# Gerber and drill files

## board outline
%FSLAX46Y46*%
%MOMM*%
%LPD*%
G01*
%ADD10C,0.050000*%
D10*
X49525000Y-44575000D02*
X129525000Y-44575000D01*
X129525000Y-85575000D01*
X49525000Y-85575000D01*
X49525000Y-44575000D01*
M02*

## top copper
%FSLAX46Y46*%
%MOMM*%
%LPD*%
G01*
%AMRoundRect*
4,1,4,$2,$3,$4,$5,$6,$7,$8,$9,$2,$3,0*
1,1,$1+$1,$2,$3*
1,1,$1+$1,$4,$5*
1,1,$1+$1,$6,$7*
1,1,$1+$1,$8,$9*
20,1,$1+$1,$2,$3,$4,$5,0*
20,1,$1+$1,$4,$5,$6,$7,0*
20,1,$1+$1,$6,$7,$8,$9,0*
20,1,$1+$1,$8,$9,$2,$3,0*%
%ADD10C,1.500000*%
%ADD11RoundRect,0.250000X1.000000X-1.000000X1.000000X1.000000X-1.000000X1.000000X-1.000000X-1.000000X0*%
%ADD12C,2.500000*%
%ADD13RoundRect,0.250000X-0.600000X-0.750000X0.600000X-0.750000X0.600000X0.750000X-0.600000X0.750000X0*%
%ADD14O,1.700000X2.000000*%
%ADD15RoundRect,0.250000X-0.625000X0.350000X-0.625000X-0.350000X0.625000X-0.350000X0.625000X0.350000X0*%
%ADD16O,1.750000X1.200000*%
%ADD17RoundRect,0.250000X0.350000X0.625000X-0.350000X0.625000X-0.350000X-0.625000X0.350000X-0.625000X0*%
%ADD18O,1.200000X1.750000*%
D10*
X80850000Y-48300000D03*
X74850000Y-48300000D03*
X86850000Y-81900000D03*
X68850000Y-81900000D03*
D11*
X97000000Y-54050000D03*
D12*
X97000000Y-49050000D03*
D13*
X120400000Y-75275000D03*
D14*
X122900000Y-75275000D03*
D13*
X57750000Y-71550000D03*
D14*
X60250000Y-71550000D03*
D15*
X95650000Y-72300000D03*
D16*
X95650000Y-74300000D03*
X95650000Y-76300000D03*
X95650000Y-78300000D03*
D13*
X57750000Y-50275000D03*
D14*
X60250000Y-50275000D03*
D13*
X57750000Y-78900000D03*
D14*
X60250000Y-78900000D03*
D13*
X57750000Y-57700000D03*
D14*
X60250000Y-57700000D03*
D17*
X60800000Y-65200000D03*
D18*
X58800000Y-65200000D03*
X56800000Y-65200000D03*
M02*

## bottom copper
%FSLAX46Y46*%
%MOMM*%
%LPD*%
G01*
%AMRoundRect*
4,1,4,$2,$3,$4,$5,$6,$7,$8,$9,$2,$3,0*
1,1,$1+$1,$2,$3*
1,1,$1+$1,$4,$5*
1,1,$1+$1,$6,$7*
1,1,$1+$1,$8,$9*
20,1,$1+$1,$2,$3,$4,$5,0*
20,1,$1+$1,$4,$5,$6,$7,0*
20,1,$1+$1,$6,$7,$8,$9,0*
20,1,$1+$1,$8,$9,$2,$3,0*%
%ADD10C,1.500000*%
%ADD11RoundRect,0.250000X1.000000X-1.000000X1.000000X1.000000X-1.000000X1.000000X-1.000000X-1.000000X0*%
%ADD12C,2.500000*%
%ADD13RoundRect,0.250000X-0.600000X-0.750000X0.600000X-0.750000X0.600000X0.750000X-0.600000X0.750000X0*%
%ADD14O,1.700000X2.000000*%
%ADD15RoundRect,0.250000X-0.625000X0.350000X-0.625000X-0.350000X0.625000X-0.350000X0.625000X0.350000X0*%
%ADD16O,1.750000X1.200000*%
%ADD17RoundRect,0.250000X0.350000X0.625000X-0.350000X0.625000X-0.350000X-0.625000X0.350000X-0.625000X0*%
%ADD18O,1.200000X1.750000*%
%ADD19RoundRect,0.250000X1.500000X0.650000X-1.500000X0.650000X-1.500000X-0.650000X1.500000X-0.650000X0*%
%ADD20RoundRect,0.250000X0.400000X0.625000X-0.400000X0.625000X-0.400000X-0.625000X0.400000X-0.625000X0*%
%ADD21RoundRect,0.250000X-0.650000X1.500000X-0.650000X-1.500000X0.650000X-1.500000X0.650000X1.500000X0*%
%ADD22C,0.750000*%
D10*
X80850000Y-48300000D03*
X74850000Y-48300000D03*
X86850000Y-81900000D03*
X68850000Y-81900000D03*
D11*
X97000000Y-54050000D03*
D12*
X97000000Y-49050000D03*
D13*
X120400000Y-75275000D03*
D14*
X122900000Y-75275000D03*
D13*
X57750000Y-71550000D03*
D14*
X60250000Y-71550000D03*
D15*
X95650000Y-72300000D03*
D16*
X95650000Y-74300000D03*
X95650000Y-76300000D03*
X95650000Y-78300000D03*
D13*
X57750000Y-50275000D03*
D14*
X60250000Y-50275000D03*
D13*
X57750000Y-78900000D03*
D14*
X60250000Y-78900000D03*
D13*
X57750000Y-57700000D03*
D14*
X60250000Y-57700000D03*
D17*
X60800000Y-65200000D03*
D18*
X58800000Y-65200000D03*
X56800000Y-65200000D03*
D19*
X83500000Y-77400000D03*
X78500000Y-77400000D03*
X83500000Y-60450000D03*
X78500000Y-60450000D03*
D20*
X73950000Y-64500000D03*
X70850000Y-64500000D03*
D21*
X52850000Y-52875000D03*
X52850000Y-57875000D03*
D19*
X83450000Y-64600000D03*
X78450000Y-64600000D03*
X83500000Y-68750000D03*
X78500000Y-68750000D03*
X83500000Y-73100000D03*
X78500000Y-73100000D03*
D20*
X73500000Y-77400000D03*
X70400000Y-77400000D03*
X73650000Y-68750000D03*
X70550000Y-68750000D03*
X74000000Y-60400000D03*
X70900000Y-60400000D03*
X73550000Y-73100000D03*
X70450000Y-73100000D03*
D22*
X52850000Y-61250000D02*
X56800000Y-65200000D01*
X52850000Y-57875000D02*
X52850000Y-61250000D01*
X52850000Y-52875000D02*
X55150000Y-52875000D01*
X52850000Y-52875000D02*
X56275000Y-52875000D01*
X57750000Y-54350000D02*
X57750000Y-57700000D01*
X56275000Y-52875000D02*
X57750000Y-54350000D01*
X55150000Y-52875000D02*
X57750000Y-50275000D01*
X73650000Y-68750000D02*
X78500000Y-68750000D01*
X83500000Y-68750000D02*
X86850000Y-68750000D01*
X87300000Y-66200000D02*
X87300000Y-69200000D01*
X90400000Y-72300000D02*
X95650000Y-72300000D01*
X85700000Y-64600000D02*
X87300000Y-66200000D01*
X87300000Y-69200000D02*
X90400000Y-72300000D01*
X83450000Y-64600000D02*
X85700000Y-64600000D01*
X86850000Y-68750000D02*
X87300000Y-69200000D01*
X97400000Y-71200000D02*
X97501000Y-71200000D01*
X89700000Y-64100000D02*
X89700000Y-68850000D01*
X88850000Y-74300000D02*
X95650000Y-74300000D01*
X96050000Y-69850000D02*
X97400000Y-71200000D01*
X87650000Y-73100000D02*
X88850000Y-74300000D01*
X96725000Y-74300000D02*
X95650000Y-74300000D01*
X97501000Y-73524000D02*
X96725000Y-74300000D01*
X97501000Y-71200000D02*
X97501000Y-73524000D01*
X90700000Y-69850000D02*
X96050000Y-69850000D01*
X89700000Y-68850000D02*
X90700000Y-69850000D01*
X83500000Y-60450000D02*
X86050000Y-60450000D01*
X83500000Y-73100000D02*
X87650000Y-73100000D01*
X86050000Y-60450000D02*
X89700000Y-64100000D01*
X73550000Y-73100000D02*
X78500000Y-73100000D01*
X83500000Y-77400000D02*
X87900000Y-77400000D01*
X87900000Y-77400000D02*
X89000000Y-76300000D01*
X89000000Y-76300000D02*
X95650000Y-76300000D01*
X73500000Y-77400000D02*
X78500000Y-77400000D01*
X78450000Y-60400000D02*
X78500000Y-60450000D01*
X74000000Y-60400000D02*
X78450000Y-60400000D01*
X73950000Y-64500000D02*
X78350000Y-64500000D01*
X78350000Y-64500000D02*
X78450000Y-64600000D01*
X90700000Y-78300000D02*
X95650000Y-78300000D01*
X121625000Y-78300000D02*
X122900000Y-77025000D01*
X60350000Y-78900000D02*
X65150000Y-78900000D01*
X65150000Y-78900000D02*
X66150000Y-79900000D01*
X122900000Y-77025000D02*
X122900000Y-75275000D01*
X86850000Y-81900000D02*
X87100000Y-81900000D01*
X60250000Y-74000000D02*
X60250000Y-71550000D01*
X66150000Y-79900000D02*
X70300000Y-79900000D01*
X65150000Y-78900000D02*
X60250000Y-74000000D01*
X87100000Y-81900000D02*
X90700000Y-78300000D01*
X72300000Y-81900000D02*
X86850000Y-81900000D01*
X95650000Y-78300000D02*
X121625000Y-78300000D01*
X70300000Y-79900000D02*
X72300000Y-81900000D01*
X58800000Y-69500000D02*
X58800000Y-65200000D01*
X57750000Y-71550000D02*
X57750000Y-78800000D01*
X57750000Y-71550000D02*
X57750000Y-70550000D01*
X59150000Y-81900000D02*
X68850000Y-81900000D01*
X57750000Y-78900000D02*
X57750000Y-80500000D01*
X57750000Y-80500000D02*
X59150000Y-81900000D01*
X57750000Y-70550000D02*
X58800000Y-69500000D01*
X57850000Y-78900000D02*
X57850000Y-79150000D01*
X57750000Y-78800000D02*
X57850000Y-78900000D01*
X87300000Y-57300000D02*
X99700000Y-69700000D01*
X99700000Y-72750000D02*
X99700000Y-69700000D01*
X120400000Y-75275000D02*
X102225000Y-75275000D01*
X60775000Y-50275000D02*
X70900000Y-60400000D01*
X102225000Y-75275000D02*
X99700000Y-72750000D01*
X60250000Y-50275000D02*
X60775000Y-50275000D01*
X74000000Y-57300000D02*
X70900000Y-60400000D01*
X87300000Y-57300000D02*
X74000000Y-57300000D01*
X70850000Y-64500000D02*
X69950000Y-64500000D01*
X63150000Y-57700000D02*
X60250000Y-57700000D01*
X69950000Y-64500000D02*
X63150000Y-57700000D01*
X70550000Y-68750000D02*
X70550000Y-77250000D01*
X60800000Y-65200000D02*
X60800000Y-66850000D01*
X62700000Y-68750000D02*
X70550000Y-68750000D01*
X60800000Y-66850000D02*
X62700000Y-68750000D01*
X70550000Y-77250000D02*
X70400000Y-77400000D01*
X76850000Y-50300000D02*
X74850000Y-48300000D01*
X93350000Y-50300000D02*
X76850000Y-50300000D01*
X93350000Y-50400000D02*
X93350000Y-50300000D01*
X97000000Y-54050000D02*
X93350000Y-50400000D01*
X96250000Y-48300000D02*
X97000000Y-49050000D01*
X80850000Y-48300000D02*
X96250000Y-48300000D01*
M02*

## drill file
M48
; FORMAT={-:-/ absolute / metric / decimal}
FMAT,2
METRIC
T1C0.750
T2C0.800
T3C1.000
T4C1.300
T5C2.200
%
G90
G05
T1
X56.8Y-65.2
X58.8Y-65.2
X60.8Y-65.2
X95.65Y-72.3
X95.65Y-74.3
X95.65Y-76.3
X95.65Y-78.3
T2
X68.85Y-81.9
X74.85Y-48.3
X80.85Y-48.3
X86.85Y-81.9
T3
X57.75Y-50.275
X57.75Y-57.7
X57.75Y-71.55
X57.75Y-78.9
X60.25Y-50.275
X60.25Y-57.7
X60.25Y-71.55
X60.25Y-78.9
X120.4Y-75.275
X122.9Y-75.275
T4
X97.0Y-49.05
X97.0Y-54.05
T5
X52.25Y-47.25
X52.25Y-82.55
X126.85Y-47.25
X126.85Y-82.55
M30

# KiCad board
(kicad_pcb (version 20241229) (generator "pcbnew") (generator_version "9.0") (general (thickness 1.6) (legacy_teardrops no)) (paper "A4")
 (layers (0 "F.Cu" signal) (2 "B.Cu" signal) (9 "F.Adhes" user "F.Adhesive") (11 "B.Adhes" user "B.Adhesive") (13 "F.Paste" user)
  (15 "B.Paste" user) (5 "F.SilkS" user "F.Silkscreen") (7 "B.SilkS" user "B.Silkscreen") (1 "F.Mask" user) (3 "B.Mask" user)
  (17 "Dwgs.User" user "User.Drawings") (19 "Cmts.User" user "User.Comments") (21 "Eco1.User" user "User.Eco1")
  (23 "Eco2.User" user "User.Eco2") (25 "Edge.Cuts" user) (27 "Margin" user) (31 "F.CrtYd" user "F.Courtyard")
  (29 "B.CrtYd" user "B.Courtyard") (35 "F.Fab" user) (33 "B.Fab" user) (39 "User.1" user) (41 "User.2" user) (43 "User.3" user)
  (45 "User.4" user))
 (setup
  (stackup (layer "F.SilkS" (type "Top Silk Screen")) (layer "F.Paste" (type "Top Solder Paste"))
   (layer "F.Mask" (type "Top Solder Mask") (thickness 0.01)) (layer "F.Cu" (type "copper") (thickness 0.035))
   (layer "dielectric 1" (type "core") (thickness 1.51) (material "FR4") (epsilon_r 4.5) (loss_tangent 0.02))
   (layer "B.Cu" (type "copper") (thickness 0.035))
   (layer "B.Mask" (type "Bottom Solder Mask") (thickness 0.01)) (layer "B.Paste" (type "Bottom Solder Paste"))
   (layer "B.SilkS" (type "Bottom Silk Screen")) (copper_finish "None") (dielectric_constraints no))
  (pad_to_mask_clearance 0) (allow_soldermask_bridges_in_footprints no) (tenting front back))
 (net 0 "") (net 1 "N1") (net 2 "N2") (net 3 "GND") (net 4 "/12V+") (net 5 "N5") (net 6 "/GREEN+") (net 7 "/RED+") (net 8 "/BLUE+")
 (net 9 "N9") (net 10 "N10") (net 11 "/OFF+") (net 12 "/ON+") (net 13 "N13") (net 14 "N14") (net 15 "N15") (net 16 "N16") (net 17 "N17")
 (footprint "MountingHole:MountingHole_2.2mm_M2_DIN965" (layer "F.Cu") (at 52.25 47.25)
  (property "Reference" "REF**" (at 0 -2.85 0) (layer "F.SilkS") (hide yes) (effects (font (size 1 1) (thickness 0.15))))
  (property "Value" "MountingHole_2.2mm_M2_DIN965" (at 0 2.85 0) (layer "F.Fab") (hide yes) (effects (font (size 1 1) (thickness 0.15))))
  (pad "" np_thru_hole circle (at 0 0) (size 2.2 2.2) (drill 2.2) (layers "*.Cu" "*.Mask")))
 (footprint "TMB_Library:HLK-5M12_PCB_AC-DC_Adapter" (layer "F.Cu") (at 77.85 65.1 -90)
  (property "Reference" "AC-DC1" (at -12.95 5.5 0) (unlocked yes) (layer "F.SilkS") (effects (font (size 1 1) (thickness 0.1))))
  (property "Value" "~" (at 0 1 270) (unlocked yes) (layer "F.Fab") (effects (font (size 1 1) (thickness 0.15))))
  (pad "1" thru_hole circle (at -16.8 -3 270) (size 1.5 1.5) (drill 0.8) (layers "*.Cu" "*.Mask") (remove_unused_layers yes)
   (keep_end_layers yes) (zone_layer_connections) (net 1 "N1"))
  (pad "2" thru_hole circle (at -16.8 3 270) (size 1.5 1.5) (drill 0.8) (layers "*.Cu" "*.Mask") (remove_unused_layers yes)
   (keep_end_layers yes) (zone_layer_connections) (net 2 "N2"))
  (pad "3" thru_hole circle (at 16.8 -9 270) (size 1.5 1.5) (drill 0.8) (layers "*.Cu" "*.Mask") (remove_unused_layers yes)
   (keep_end_layers yes) (zone_layer_connections) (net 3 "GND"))
  (pad "4" thru_hole circle (at 16.8 9 270) (size 1.5 1.5) (drill 0.8) (layers "*.Cu" "*.Mask") (remove_unused_layers yes)
   (keep_end_layers yes) (zone_layer_connections) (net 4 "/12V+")))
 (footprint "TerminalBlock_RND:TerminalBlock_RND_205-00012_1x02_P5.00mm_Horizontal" (layer "F.Cu") (at 97 54.05 90)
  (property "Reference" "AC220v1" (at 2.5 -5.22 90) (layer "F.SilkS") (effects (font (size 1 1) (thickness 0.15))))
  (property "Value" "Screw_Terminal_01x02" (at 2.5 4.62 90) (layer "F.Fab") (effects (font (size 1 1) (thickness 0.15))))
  (pad "1" thru_hole roundrect (at 0 0 90) (size 2.5 2.5) (drill 1.3) (layers "*.Cu" "*.Mask") (remove_unused_layers no)
   (roundrect_rratio 0.1) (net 2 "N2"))
  (pad "2" thru_hole circle (at 5 0 90) (size 2.5 2.5) (drill 1.3) (layers "*.Cu" "*.Mask") (remove_unused_layers no) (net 1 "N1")))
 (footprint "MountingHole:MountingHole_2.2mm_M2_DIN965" (layer "F.Cu") (at 52.25 82.55)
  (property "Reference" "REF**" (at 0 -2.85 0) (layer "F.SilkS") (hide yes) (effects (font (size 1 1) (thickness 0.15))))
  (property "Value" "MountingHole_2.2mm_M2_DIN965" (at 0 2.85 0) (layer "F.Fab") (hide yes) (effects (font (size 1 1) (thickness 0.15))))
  (pad "" np_thru_hole circle (at 0 0) (size 2.2 2.2) (drill 2.2) (layers "*.Cu" "*.Mask")))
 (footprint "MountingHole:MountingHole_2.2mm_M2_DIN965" (layer "F.Cu") (at 126.85 82.55)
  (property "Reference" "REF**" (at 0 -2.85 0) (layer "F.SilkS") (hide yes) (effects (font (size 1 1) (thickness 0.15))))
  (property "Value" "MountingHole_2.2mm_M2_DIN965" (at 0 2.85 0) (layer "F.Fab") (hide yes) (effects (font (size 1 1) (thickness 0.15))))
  (pad "" np_thru_hole circle (at 0 0) (size 2.2 2.2) (drill 2.2) (layers "*.Cu" "*.Mask")))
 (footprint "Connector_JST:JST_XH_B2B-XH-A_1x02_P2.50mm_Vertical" (layer "F.Cu") (at 120.4 75.275)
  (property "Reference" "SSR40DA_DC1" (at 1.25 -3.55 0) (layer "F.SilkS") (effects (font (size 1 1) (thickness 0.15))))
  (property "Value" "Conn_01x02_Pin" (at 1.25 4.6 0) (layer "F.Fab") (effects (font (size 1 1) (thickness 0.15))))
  (pad "1" thru_hole roundrect (at 0 0) (size 1.7 2) (drill 1) (layers "*.Cu" "*.Mask") (remove_unused_layers no)
   (roundrect_rratio 0.147059) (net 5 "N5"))
  (pad "2" thru_hole oval (at 2.5 0) (size 1.7 2) (drill 1) (layers "*.Cu" "*.Mask") (remove_unused_layers no) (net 3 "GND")))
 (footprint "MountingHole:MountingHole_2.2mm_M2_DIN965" (layer "F.Cu") (at 126.85 47.25)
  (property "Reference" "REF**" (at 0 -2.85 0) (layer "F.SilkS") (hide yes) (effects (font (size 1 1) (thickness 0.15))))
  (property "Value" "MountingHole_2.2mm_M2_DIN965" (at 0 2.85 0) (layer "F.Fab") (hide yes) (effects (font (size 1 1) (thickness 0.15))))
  (pad "" np_thru_hole circle (at 0 0) (size 2.2 2.2) (drill 2.2) (layers "*.Cu" "*.Mask")))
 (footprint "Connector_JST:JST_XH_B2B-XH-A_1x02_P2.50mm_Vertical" (layer "F.Cu") (at 57.75 71.55)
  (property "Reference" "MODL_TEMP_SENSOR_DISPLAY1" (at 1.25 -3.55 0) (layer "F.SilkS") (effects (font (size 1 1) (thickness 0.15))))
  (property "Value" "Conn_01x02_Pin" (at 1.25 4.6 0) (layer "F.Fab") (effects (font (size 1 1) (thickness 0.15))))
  (pad "1" thru_hole roundrect (at 0 0) (size 1.7 2) (drill 1) (layers "*.Cu" "*.Mask") (remove_unused_layers no)
   (roundrect_rratio 0.147059) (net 4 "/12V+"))
  (pad "2" thru_hole oval (at 2.5 0) (size 1.7 2) (drill 1) (layers "*.Cu" "*.Mask") (remove_unused_layers no) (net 3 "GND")))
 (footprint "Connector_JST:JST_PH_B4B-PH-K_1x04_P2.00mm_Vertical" (layer "F.Cu") (at 95.65 72.3 -90)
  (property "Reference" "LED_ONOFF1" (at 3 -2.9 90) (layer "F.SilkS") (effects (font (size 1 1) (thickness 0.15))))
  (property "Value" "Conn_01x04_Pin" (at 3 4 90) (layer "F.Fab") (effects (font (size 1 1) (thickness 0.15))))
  (pad "1" thru_hole roundrect (at 0 0 270) (size 1.2 1.75) (drill 0.75) (layers "*.Cu" "*.Mask") (remove_unused_layers no)
   (roundrect_rratio 0.208333) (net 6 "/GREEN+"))
  (pad "2" thru_hole oval (at 2 0 270) (size 1.2 1.75) (drill 0.75) (layers "*.Cu" "*.Mask") (remove_unused_layers no) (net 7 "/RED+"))
  (pad "3" thru_hole oval (at 4 0 270) (size 1.2 1.75) (drill 0.75) (layers "*.Cu" "*.Mask") (remove_unused_layers no) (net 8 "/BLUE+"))
  (pad "4" thru_hole oval (at 6 0 270) (size 1.2 1.75) (drill 0.75) (layers "*.Cu" "*.Mask") (remove_unused_layers no) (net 3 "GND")))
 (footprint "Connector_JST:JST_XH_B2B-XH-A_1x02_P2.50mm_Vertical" (layer "F.Cu") (at 57.75 50.275)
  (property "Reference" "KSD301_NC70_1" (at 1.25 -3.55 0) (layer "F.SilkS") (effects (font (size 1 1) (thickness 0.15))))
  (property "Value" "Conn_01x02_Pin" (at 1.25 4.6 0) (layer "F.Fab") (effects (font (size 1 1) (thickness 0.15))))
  (pad "1" thru_hole roundrect (at 0 0) (size 1.7 2) (drill 1) (layers "*.Cu" "*.Mask") (remove_unused_layers no)
   (roundrect_rratio 0.147059) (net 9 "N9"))
  (pad "2" thru_hole oval (at 2.5 0) (size 1.7 2) (drill 1) (layers "*.Cu" "*.Mask") (remove_unused_layers no) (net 5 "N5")))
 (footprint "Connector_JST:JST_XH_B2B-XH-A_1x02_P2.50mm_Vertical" (layer "F.Cu") (at 57.75 78.9)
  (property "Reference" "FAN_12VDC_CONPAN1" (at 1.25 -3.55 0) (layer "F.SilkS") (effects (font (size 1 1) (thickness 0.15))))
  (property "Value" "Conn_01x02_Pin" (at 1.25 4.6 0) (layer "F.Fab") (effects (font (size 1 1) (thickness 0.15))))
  (pad "1" thru_hole roundrect (at 0 0) (size 1.7 2) (drill 1) (layers "*.Cu" "*.Mask") (remove_unused_layers no)
   (roundrect_rratio 0.147059) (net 4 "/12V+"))
  (pad "2" thru_hole oval (at 2.5 0) (size 1.7 2) (drill 1) (layers "*.Cu" "*.Mask") (remove_unused_layers no) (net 3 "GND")))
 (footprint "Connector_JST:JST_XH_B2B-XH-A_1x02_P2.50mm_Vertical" (layer "F.Cu") (at 57.75 57.7)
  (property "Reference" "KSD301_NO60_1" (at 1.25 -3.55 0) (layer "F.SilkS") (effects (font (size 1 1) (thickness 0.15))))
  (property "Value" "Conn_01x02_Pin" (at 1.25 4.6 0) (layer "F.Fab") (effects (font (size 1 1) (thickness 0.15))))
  (pad "1" thru_hole roundrect (at 0 0) (size 1.7 2) (drill 1) (layers "*.Cu" "*.Mask") (remove_unused_layers no)
   (roundrect_rratio 0.147059) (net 9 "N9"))
  (pad "2" thru_hole oval (at 2.5 0) (size 1.7 2) (drill 1) (layers "*.Cu" "*.Mask") (remove_unused_layers no) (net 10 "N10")))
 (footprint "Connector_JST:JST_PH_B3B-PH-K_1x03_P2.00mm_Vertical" (layer "F.Cu") (at 60.8 65.2 180)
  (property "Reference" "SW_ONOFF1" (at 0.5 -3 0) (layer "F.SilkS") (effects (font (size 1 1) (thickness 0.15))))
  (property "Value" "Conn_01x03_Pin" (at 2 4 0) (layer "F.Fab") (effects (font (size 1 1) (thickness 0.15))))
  (pad "1" thru_hole roundrect (at 0 0 180) (size 1.2 1.75) (drill 0.75) (layers "*.Cu" "*.Mask") (remove_unused_layers no)
   (roundrect_rratio 0.208333) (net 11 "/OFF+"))
  (pad "2" thru_hole oval (at 2 0 180) (size 1.2 1.75) (drill 0.75) (layers "*.Cu" "*.Mask") (remove_unused_layers no) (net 4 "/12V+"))
  (pad "3" thru_hole oval (at 4 0 180) (size 1.2 1.75) (drill 0.75) (layers "*.Cu" "*.Mask") (remove_unused_layers no) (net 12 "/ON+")))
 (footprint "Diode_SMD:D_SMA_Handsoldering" (layer "B.Cu") (at 81 77.4 180)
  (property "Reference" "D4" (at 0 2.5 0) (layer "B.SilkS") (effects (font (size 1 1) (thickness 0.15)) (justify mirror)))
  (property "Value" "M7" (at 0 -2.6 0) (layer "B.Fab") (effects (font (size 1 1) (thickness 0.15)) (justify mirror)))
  (pad "1" smd roundrect (at -2.5 0 180) (size 3.5 1.8) (layers "B.Cu" "B.Mask" "B.Paste") (roundrect_rratio 0.1388888889) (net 8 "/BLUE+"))
  (pad "2" smd roundrect (at 2.5 0 180) (size 3.5 1.8) (layers "B.Cu" "B.Mask" "B.Paste") (roundrect_rratio 0.1388888889) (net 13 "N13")))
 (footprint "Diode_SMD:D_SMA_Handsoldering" (layer "B.Cu") (at 81 60.45 180)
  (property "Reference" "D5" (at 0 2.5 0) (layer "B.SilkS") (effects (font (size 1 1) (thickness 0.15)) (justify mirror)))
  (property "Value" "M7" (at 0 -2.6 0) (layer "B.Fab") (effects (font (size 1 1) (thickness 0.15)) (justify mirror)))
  (pad "1" smd roundrect (at -2.5 0 180) (size 3.5 1.8) (layers "B.Cu" "B.Mask" "B.Paste") (roundrect_rratio 0.1388888889) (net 7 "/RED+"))
  (pad "2" smd roundrect (at 2.5 0 180) (size 3.5 1.8) (layers "B.Cu" "B.Mask" "B.Paste") (roundrect_rratio 0.1388888889) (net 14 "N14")))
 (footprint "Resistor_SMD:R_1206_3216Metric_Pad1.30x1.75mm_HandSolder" (layer "B.Cu") (at 72.4 64.5 180)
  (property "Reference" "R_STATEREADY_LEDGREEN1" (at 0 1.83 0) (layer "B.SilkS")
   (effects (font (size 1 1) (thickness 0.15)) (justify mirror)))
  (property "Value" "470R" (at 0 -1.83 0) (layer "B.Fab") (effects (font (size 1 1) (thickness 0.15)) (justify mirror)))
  (pad "1" smd roundrect (at -1.55 0 180) (size 1.3 1.75) (layers "B.Cu" "B.Mask" "B.Paste") (roundrect_rratio 0.192308) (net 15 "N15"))
  (pad "2" smd roundrect (at 1.55 0 180) (size 1.3 1.75) (layers "B.Cu" "B.Mask" "B.Paste") (roundrect_rratio 0.192308) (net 10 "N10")))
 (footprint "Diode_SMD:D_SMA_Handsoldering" (layer "B.Cu") (at 52.85 55.375 -90)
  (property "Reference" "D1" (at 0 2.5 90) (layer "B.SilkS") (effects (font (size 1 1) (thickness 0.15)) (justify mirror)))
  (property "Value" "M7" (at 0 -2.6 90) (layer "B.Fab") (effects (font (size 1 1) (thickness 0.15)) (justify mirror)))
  (pad "1" smd roundrect (at -2.5 0 270) (size 3.5 1.8) (layers "B.Cu" "B.Mask" "B.Paste") (roundrect_rratio 0.1388888889) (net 9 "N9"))
  (pad "2" smd roundrect (at 2.5 0 270) (size 3.5 1.8) (layers "B.Cu" "B.Mask" "B.Paste") (roundrect_rratio 0.1388888889) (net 12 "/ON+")))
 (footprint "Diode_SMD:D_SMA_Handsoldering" (layer "B.Cu") (at 80.95 64.6 180)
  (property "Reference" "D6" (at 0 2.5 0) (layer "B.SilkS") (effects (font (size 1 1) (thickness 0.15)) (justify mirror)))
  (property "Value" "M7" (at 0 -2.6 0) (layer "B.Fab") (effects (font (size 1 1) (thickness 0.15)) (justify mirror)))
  (pad "1" smd roundrect (at -2.5 0 180) (size 3.5 1.8) (layers "B.Cu" "B.Mask" "B.Paste") (roundrect_rratio 0.1388888889) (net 6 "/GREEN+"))
  (pad "2" smd roundrect (at 2.5 0 180) (size 3.5 1.8) (layers "B.Cu" "B.Mask" "B.Paste") (roundrect_rratio 0.1388888889) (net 15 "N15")))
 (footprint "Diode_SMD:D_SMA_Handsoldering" (layer "B.Cu") (at 81 68.75 180)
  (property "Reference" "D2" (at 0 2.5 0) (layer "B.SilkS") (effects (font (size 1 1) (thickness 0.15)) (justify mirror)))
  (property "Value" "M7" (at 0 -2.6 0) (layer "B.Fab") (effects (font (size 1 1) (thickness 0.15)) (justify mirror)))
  (pad "1" smd roundrect (at -2.5 0 180) (size 3.5 1.8) (layers "B.Cu" "B.Mask" "B.Paste") (roundrect_rratio 0.1388888889) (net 6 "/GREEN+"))
  (pad "2" smd roundrect (at 2.5 0 180) (size 3.5 1.8) (layers "B.Cu" "B.Mask" "B.Paste") (roundrect_rratio 0.1388888889) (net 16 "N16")))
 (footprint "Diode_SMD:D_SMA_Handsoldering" (layer "B.Cu") (at 81 73.1 180)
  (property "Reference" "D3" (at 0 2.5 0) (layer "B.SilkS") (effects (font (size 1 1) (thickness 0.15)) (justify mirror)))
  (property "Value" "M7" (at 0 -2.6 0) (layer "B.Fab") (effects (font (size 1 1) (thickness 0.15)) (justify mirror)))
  (pad "1" smd roundrect (at -2.5 0 180) (size 3.5 1.8) (layers "B.Cu" "B.Mask" "B.Paste") (roundrect_rratio 0.1388888889) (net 7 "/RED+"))
  (pad "2" smd roundrect (at 2.5 0 180) (size 3.5 1.8) (layers "B.Cu" "B.Mask" "B.Paste") (roundrect_rratio 0.1388888889) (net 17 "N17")))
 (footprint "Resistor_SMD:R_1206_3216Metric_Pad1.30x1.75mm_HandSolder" (layer "B.Cu") (at 71.95 77.4 180)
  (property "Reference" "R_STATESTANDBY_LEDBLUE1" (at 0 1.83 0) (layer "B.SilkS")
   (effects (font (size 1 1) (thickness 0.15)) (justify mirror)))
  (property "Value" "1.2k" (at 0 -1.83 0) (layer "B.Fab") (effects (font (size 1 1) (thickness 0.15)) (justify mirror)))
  (pad "1" smd roundrect (at -1.55 0 180) (size 1.3 1.75) (layers "B.Cu" "B.Mask" "B.Paste") (roundrect_rratio 0.192308) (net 13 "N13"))
  (pad "2" smd roundrect (at 1.55 0 180) (size 1.3 1.75) (layers "B.Cu" "B.Mask" "B.Paste") (roundrect_rratio 0.192308) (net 11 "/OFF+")))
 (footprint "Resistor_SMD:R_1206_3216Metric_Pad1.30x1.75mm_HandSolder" (layer "B.Cu") (at 72.1 68.75 180)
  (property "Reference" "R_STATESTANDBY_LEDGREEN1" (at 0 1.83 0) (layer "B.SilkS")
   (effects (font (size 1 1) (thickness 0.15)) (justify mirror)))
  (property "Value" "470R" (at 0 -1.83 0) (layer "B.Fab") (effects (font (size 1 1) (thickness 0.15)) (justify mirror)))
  (pad "1" smd roundrect (at -1.55 0 180) (size 1.3 1.75) (layers "B.Cu" "B.Mask" "B.Paste") (roundrect_rratio 0.192308) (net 16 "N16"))
  (pad "2" smd roundrect (at 1.55 0 180) (size 1.3 1.75) (layers "B.Cu" "B.Mask" "B.Paste") (roundrect_rratio 0.192308) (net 11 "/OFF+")))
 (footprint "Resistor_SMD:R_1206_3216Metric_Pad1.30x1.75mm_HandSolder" (layer "B.Cu") (at 72.45 60.4 180)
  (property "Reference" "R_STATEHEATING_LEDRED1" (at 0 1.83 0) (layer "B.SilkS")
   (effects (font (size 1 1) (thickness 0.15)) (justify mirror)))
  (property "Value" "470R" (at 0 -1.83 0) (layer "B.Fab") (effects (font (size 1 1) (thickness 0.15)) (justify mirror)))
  (pad "1" smd roundrect (at -1.55 0 180) (size 1.3 1.75) (layers "B.Cu" "B.Mask" "B.Paste") (roundrect_rratio 0.192308) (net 14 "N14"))
  (pad "2" smd roundrect (at 1.55 0 180) (size 1.3 1.75) (layers "B.Cu" "B.Mask" "B.Paste") (roundrect_rratio 0.192308) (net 5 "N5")))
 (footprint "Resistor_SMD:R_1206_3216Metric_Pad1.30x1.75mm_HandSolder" (layer "B.Cu") (at 72 73.1 180)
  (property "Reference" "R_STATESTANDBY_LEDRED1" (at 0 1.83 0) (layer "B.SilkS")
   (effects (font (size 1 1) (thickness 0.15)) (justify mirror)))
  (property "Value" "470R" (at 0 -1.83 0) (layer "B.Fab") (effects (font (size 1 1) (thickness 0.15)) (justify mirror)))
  (pad "1" smd roundrect (at -1.55 0 180) (size 1.3 1.75) (layers "B.Cu" "B.Mask" "B.Paste") (roundrect_rratio 0.192308) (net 17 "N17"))
  (pad "2" smd roundrect (at 1.55 0 180) (size 1.3 1.75) (layers "B.Cu" "B.Mask" "B.Paste") (roundrect_rratio 0.192308) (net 11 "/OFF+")))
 (gr_rect (start 49.525 44.575) (end 129.525 85.575) (stroke (width 0.05) (type solid)) (fill no) (layer "Edge.Cuts"))
 (segment (start 52.85 61.25) (end 56.8 65.2) (width 0.75) (layer "B.Cu") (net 12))
 (segment (start 52.85 57.875) (end 52.85 61.25) (width 0.75) (layer "B.Cu") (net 12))
 (segment (start 52.85 52.875) (end 55.15 52.875) (width 0.75) (layer "B.Cu") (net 9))
 (segment (start 52.85 52.875) (end 56.275 52.875) (width 0.75) (layer "B.Cu") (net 9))
 (segment (start 57.75 54.35) (end 57.75 57.7) (width 0.75) (layer "B.Cu") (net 9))
 (segment (start 56.275 52.875) (end 57.75 54.35) (width 0.75) (layer "B.Cu") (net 9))
 (segment (start 55.15 52.875) (end 57.75 50.275) (width 0.75) (layer "B.Cu") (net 9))
 (segment (start 73.65 68.75) (end 78.5 68.75) (width 0.75) (layer "B.Cu") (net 16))
 (segment (start 83.5 68.75) (end 86.85 68.75) (width 0.75) (layer "B.Cu") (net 6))
 (segment (start 87.3 66.2) (end 87.3 69.2) (width 0.75) (layer "B.Cu") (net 6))
 (segment (start 90.4 72.3) (end 95.65 72.3) (width 0.75) (layer "B.Cu") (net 6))
 (segment (start 85.7 64.6) (end 87.3 66.2) (width 0.75) (layer "B.Cu") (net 6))
 (segment (start 87.3 69.2) (end 90.4 72.3) (width 0.75) (layer "B.Cu") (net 6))
 (segment (start 83.45 64.6) (end 85.7 64.6) (width 0.75) (layer "B.Cu") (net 6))
 (segment (start 86.85 68.75) (end 87.3 69.2) (width 0.75) (layer "B.Cu") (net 6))
 (segment (start 97.4 71.2) (end 97.501 71.2) (width 0.75) (layer "B.Cu") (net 7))
 (segment (start 89.7 64.1) (end 89.7 68.85) (width 0.75) (layer "B.Cu") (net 7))
 (segment (start 88.85 74.3) (end 95.65 74.3) (width 0.75) (layer "B.Cu") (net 7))
 (segment (start 96.05 69.85) (end 97.4 71.2) (width 0.75) (layer "B.Cu") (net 7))
 (segment (start 87.65 73.1) (end 88.85 74.3) (width 0.75) (layer "B.Cu") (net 7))
 (segment (start 96.725 74.3) (end 95.65 74.3) (width 0.75) (layer "B.Cu") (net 7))
 (segment (start 97.501 73.524) (end 96.725 74.3) (width 0.75) (layer "B.Cu") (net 7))
 (segment (start 97.501 71.2) (end 97.501 73.524) (width 0.75) (layer "B.Cu") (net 7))
 (segment (start 90.7 69.85) (end 96.05 69.85) (width 0.75) (layer "B.Cu") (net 7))
 (segment (start 89.7 68.85) (end 90.7 69.85) (width 0.75) (layer "B.Cu") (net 7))
 (segment (start 83.5 60.45) (end 86.05 60.45) (width 0.75) (layer "B.Cu") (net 7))
 (segment (start 83.5 73.1) (end 87.65 73.1) (width 0.75) (layer "B.Cu") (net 7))
 (segment (start 86.05 60.45) (end 89.7 64.1) (width 0.75) (layer "B.Cu") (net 7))
 (segment (start 73.55 73.1) (end 78.5 73.1) (width 0.75) (layer "B.Cu") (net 17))
 (segment (start 83.5 77.4) (end 87.9 77.4) (width 0.75) (layer "B.Cu") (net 8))
 (segment (start 87.9 77.4) (end 89 76.3) (width 0.75) (layer "B.Cu") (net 8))
 (segment (start 89 76.3) (end 95.65 76.3) (width 0.75) (layer "B.Cu") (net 8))
 (segment (start 73.5 77.4) (end 78.5 77.4) (width 0.75) (layer "B.Cu") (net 13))
 (segment (start 78.45 60.4) (end 78.5 60.45) (width 0.75) (layer "B.Cu") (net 14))
 (segment (start 74 60.4) (end 78.45 60.4) (width 0.75) (layer "B.Cu") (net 14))
 (segment (start 73.95 64.5) (end 78.35 64.5) (width 0.75) (layer "B.Cu") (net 15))
 (segment (start 78.35 64.5) (end 78.45 64.6) (width 0.75) (layer "B.Cu") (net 15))
 (segment (start 90.7 78.3) (end 95.65 78.3) (width 0.75) (layer "B.Cu") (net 3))
 (segment (start 121.625 78.3) (end 122.9 77.025) (width 0.75) (layer "B.Cu") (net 3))
 (segment (start 60.35 78.9) (end 65.15 78.9) (width 0.75) (layer "B.Cu") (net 3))
 (segment (start 65.15 78.9) (end 66.15 79.9) (width 0.75) (layer "B.Cu") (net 3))
 (segment (start 122.9 77.025) (end 122.9 75.275) (width 0.75) (layer "B.Cu") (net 3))
 (segment (start 86.85 81.9) (end 87.1 81.9) (width 0.75) (layer "B.Cu") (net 3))
 (segment (start 60.25 74) (end 60.25 71.55) (width 0.75) (layer "B.Cu") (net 3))
 (segment (start 66.15 79.9) (end 70.3 79.9) (width 0.75) (layer "B.Cu") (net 3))
 (segment (start 65.15 78.9) (end 60.25 74) (width 0.75) (layer "B.Cu") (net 3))
 (segment (start 87.1 81.9) (end 90.7 78.3) (width 0.75) (layer "B.Cu") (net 3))
 (segment (start 72.3 81.9) (end 86.85 81.9) (width 0.75) (layer "B.Cu") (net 3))
 (segment (start 95.65 78.3) (end 121.625 78.3) (width 0.75) (layer "B.Cu") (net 3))
 (segment (start 70.3 79.9) (end 72.3 81.9) (width 0.75) (layer "B.Cu") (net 3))
 (segment (start 58.8 69.5) (end 58.8 65.2) (width 0.75) (layer "B.Cu") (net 4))
 (segment (start 57.75 71.55) (end 57.75 78.8) (width 0.75) (layer "B.Cu") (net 4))
 (segment (start 57.75 71.55) (end 57.75 70.55) (width 0.75) (layer "B.Cu") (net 4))
 (segment (start 59.15 81.9) (end 68.85 81.9) (width 0.75) (layer "B.Cu") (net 4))
 (segment (start 57.75 78.9) (end 57.75 80.5) (width 0.75) (layer "B.Cu") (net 4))
 (segment (start 57.75 80.5) (end 59.15 81.9) (width 0.75) (layer "B.Cu") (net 4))
 (segment (start 57.75 70.55) (end 58.8 69.5) (width 0.75) (layer "B.Cu") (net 4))
 (segment (start 57.85 78.9) (end 57.85 79.15) (width 0.75) (layer "B.Cu") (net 4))
 (segment (start 57.75 78.8) (end 57.85 78.9) (width 0.75) (layer "B.Cu") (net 4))
 (segment (start 87.3 57.3) (end 99.7 69.7) (width 0.75) (layer "B.Cu") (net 5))
 (segment (start 99.7 72.75) (end 99.7 69.7) (width 0.75) (layer "B.Cu") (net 5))
 (segment (start 120.4 75.275) (end 102.225 75.275) (width 0.75) (layer "B.Cu") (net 5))
 (segment (start 60.775 50.275) (end 70.9 60.4) (width 0.75) (layer "B.Cu") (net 5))
 (segment (start 102.225 75.275) (end 99.7 72.75) (width 0.75) (layer "B.Cu") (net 5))
 (segment (start 60.25 50.275) (end 60.775 50.275) (width 0.75) (layer "B.Cu") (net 5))
 (segment (start 74 57.3) (end 70.9 60.4) (width 0.75) (layer "B.Cu") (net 5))
 (segment (start 87.3 57.3) (end 74 57.3) (width 0.75) (layer "B.Cu") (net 5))
 (segment (start 70.85 64.5) (end 69.95 64.5) (width 0.75) (layer "B.Cu") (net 10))
 (segment (start 63.15 57.7) (end 60.25 57.7) (width 0.75) (layer "B.Cu") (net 10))
 (segment (start 69.95 64.5) (end 63.15 57.7) (width 0.75) (layer "B.Cu") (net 10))
 (segment (start 70.55 68.75) (end 70.55 77.25) (width 0.75) (layer "B.Cu") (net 11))
 (segment (start 60.8 65.2) (end 60.8 66.85) (width 0.75) (layer "B.Cu") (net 11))
 (segment (start 62.7 68.75) (end 70.55 68.75) (width 0.75) (layer "B.Cu") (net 11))
 (segment (start 60.8 66.85) (end 62.7 68.75) (width 0.75) (layer "B.Cu") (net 11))
 (segment (start 70.55 77.25) (end 70.4 77.4) (width 0.75) (layer "B.Cu") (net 11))
 (segment (start 76.85 50.3) (end 74.85 48.3) (width 0.75) (layer "B.Cu") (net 2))
 (segment (start 93.35 50.3) (end 76.85 50.3) (width 0.75) (layer "B.Cu") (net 2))
 (segment (start 93.35 50.4) (end 93.35 50.3) (width 0.75) (layer "B.Cu") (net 2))
 (segment (start 97 54.05) (end 93.35 50.4) (width 0.75) (layer "B.Cu") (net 2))
 (segment (start 96.25 48.3) (end 97 49.05) (width 0.75) (layer "B.Cu") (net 1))
 (segment (start 80.85 48.3) (end 96.25 48.3) (width 0.75) (layer "B.Cu") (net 1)))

